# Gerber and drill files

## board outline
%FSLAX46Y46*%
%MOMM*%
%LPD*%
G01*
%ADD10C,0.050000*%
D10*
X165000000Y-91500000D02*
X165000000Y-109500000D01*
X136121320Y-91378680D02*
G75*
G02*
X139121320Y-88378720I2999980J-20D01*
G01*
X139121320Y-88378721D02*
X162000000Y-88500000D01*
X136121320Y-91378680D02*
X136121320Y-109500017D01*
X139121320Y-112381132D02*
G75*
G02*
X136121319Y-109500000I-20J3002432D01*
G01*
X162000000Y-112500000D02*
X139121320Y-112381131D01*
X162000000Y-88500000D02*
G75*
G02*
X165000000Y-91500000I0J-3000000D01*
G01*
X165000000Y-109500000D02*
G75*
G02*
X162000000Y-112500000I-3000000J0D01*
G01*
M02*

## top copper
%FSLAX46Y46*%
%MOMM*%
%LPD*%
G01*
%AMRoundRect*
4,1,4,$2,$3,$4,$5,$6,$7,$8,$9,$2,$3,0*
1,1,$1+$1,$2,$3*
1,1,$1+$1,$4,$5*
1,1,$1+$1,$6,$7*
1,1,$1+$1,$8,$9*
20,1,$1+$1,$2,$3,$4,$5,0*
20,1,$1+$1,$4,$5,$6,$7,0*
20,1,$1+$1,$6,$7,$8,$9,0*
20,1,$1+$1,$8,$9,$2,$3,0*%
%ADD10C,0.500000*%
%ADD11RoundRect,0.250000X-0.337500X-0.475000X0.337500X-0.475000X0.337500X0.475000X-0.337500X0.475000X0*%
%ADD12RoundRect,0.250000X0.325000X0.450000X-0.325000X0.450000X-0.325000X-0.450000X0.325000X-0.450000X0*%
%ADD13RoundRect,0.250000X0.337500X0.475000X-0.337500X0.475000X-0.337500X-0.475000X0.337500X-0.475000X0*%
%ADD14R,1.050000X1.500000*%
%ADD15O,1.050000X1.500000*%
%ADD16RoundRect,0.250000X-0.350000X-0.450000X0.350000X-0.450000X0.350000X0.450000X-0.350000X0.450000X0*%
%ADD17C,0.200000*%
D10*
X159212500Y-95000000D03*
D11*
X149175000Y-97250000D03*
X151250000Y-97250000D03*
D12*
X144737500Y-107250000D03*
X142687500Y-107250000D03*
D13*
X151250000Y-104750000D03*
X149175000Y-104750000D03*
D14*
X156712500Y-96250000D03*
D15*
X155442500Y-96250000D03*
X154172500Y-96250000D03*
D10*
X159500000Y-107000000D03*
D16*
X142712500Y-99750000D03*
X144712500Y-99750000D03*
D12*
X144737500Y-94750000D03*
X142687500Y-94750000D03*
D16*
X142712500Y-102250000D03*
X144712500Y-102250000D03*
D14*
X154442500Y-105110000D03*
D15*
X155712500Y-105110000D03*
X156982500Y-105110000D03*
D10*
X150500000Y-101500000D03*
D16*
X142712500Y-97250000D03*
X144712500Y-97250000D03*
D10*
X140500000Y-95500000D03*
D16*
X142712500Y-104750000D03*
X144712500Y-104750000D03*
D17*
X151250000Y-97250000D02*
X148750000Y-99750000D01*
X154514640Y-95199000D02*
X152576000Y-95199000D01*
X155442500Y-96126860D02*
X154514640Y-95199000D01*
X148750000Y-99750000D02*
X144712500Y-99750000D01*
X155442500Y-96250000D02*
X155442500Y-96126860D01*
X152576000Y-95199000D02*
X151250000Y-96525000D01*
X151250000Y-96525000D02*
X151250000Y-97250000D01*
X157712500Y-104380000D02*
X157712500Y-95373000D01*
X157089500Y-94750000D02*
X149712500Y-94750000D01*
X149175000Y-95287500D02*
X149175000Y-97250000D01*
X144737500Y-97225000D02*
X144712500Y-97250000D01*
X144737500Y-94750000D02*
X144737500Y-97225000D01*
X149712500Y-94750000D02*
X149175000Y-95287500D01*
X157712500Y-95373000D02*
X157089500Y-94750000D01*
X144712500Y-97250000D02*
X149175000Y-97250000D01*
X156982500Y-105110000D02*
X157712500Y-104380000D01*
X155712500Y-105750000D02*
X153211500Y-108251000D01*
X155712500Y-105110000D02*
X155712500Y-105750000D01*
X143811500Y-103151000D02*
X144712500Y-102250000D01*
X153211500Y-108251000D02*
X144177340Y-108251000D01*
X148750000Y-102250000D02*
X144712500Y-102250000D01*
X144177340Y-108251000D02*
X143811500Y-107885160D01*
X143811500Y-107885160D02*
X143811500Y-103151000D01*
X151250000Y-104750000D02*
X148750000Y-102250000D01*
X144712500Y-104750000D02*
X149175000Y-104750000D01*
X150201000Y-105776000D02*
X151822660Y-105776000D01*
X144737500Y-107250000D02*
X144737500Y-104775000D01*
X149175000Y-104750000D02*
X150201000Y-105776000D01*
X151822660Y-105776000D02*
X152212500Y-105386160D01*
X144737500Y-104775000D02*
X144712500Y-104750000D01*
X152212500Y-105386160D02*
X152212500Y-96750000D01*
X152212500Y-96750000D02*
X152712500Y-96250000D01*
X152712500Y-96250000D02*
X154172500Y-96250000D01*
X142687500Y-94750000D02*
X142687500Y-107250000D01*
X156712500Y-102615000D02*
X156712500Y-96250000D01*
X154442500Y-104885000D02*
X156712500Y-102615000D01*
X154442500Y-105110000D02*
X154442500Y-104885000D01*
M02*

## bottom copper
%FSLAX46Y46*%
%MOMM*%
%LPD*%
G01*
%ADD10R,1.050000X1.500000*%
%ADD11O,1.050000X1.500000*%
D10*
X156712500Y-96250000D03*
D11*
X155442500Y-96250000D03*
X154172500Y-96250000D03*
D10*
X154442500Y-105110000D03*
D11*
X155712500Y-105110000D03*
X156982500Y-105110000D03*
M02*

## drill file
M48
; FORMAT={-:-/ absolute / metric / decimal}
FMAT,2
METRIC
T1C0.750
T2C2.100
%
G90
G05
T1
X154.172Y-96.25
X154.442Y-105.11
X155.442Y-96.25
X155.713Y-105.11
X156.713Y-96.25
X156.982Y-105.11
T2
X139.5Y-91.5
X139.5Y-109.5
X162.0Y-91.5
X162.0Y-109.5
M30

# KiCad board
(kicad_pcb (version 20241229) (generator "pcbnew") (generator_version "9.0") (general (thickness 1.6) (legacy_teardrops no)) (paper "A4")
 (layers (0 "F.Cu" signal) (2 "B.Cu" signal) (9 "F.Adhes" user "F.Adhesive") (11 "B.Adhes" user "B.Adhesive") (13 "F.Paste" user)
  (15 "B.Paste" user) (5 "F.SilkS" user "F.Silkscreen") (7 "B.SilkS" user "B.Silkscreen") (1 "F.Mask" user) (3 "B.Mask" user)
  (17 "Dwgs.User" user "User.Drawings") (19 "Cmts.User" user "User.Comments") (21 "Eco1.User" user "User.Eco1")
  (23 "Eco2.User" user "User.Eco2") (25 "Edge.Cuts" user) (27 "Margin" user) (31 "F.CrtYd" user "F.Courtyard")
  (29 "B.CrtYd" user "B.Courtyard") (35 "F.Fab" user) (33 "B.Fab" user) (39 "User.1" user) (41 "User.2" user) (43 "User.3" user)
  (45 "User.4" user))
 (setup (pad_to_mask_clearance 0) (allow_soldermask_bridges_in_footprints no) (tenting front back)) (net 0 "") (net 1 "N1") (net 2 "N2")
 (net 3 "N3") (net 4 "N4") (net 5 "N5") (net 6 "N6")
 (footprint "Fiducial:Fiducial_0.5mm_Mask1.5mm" (layer "F.Cu") (at 159.2125 95)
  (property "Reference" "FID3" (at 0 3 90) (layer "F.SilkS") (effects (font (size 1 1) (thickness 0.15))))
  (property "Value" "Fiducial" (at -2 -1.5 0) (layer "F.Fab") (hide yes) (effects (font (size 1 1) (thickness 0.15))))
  (pad "" smd circle (at 0 0) (size 0.5 0.5) (layers "F.Cu" "F.Mask") (solder_mask_margin 0.5)))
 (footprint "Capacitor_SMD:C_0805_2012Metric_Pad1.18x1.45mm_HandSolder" (layer "F.Cu") (at 150.2125 97.25)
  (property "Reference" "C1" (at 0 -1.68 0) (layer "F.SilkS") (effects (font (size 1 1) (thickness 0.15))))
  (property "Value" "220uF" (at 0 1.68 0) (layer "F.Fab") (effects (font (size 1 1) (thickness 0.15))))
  (pad "1" smd roundrect (at -1.0375 0) (size 1.175 1.45) (layers "F.Cu" "F.Mask" "F.Paste") (roundrect_rratio 0.212766) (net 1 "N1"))
  (pad "2" smd roundrect (at 1.0375 0) (size 1.175 1.45) (layers "F.Cu" "F.Mask" "F.Paste") (roundrect_rratio 0.212766) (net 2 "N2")))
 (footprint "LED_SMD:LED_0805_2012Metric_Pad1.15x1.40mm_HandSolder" (layer "F.Cu") (at 143.7125 107.25 180)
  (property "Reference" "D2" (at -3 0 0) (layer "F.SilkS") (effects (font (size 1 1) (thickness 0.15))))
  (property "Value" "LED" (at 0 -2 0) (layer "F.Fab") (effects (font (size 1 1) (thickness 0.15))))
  (pad "1" smd roundrect (at -1.025 0 180) (size 1.15 1.4) (layers "F.Cu" "F.Mask" "F.Paste") (roundrect_rratio 0.217391) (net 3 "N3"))
  (pad "2" smd roundrect (at 1.025 0 180) (size 1.15 1.4) (layers "F.Cu" "F.Mask" "F.Paste") (roundrect_rratio 0.217391) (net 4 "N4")))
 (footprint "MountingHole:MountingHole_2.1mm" (layer "F.Cu") (at 162 91.5)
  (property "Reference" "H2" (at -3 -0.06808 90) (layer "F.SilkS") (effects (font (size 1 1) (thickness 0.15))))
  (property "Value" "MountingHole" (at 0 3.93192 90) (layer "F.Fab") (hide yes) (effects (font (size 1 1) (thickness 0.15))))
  (pad "" np_thru_hole circle (at 0 0) (size 2.1 2.1) (drill 2.1) (layers "*.Cu" "*.Mask")))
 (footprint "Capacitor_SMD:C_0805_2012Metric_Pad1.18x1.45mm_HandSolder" (layer "F.Cu") (at 150.2125 104.75 180)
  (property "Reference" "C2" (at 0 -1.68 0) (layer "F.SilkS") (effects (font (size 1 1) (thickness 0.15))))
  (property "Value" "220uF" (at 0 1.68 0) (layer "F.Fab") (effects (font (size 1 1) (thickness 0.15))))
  (pad "1" smd roundrect (at -1.0375 0 180) (size 1.175 1.45) (layers "F.Cu" "F.Mask" "F.Paste") (roundrect_rratio 0.212766) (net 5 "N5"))
  (pad "2" smd roundrect (at 1.0375 0 180) (size 1.175 1.45) (layers "F.Cu" "F.Mask" "F.Paste") (roundrect_rratio 0.212766) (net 3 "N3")))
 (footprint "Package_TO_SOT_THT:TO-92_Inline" (layer "F.Cu") (at 156.7125 96.25 180)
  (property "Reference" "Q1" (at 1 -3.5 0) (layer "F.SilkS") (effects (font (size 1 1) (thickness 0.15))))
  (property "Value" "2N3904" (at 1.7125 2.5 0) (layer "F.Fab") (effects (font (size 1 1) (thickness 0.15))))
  (pad "1" thru_hole rect (at 0 0 180) (size 1.05 1.5) (drill 0.75) (layers "*.Cu" "*.Mask") (remove_unused_layers no) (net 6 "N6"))
  (pad "2" thru_hole oval (at 1.27 0 180) (size 1.05 1.5) (drill 0.75) (layers "*.Cu" "*.Mask") (remove_unused_layers no) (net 2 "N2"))
  (pad "3" thru_hole oval (at 2.54 0 180) (size 1.05 1.5) (drill 0.75) (layers "*.Cu" "*.Mask") (remove_unused_layers no) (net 3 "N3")))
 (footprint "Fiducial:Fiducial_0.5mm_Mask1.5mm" (layer "F.Cu") (at 159.5 107)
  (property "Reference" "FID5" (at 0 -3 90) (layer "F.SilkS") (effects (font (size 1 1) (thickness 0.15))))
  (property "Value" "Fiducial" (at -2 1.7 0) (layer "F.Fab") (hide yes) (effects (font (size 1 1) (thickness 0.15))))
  (pad "" smd circle (at 0 0) (size 0.5 0.5) (layers "F.Cu" "F.Mask") (solder_mask_margin 0.5)))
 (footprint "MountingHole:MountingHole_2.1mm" (layer "F.Cu") (at 139.5 109.5)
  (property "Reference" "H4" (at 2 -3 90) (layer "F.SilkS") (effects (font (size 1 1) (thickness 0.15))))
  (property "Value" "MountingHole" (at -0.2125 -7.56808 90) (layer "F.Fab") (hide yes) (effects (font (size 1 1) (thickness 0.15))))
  (pad "" np_thru_hole circle (at 0 0) (size 2.1 2.1) (drill 2.1) (layers "*.Cu" "*.Mask")))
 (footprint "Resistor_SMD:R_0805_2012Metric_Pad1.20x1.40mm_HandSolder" (layer "F.Cu") (at 143.7125 99.75)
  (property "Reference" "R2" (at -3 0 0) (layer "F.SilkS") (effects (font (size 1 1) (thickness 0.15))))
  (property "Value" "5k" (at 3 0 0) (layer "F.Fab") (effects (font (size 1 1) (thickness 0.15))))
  (pad "1" smd roundrect (at -1 0) (size 1.2 1.4) (layers "F.Cu" "F.Mask" "F.Paste") (roundrect_rratio 0.208333) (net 4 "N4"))
  (pad "2" smd roundrect (at 1 0) (size 1.2 1.4) (layers "F.Cu" "F.Mask" "F.Paste") (roundrect_rratio 0.208333) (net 2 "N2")))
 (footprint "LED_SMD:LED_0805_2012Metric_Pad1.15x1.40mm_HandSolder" (layer "F.Cu") (at 143.7125 94.75 180)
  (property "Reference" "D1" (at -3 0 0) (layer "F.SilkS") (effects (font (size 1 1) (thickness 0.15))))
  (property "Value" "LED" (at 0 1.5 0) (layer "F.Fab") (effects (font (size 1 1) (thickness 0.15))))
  (pad "1" smd roundrect (at -1.025 0 180) (size 1.15 1.4) (layers "F.Cu" "F.Mask" "F.Paste") (roundrect_rratio 0.217391) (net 1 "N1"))
  (pad "2" smd roundrect (at 1.025 0 180) (size 1.15 1.4) (layers "F.Cu" "F.Mask" "F.Paste") (roundrect_rratio 0.217391) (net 4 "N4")))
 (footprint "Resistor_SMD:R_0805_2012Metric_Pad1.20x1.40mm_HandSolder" (layer "F.Cu") (at 143.7125 102.25)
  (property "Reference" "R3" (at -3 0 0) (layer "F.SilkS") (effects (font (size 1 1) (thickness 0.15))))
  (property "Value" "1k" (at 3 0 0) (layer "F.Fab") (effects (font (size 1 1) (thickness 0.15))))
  (pad "1" smd roundrect (at -1 0) (size 1.2 1.4) (layers "F.Cu" "F.Mask" "F.Paste") (roundrect_rratio 0.208333) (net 4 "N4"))
  (pad "2" smd roundrect (at 1 0) (size 1.2 1.4) (layers "F.Cu" "F.Mask" "F.Paste") (roundrect_rratio 0.208333) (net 5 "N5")))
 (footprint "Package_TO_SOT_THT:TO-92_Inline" (layer "F.Cu") (at 154.4425 105.11)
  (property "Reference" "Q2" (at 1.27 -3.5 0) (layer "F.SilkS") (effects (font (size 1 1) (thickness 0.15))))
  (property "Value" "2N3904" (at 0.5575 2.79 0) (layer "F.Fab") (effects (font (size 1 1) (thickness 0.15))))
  (pad "1" thru_hole rect (at 0 0) (size 1.05 1.5) (drill 0.75) (layers "*.Cu" "*.Mask") (remove_unused_layers no) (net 6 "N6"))
  (pad "2" thru_hole oval (at 1.27 0) (size 1.05 1.5) (drill 0.75) (layers "*.Cu" "*.Mask") (remove_unused_layers no) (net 5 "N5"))
  (pad "3" thru_hole oval (at 2.54 0) (size 1.05 1.5) (drill 0.75) (layers "*.Cu" "*.Mask") (remove_unused_layers no) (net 1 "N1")))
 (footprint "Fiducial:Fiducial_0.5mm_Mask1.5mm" (layer "F.Cu") (at 150.5 101.5)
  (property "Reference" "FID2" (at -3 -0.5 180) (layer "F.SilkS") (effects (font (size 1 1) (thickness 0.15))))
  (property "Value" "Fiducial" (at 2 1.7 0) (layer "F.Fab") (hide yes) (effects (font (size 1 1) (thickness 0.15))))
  (pad "" smd circle (at 0 0) (size 0.5 0.5) (layers "F.Cu" "F.Mask") (solder_mask_margin 0.5)))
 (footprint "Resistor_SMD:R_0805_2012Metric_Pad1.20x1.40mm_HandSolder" (layer "F.Cu") (at 143.7125 97.25)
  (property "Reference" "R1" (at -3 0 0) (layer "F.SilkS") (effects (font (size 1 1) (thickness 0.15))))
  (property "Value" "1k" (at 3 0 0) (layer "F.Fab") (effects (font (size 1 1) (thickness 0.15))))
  (pad "1" smd roundrect (at -1 0) (size 1.2 1.4) (layers "F.Cu" "F.Mask" "F.Paste") (roundrect_rratio 0.208333) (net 4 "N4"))
  (pad "2" smd roundrect (at 1 0) (size 1.2 1.4) (layers "F.Cu" "F.Mask" "F.Paste") (roundrect_rratio 0.208333) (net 1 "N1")))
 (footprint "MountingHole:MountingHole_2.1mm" (layer "F.Cu") (at 139.5 91.5)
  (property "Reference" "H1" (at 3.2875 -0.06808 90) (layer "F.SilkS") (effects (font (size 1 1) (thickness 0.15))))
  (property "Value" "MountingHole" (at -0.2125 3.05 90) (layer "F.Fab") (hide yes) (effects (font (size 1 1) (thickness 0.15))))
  (pad "" np_thru_hole circle (at 0 0) (size 2.1 2.1) (drill 2.1) (layers "*.Cu" "*.Mask")))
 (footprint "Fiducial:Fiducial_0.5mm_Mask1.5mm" (layer "F.Cu") (at 140.5 95.5)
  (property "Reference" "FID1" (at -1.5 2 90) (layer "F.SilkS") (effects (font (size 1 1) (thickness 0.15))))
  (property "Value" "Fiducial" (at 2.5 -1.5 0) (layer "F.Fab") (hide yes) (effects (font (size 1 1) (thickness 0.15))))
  (pad "" smd circle (at 0 0) (size 0.5 0.5) (layers "F.Cu" "F.Mask") (solder_mask_margin 0.5)))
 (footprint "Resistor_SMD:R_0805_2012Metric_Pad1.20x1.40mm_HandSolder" (layer "F.Cu") (at 143.7125 104.75)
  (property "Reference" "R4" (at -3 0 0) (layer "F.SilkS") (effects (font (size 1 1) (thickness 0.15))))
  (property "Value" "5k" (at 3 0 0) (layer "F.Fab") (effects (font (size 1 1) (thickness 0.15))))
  (pad "1" smd roundrect (at -1 0) (size 1.2 1.4) (layers "F.Cu" "F.Mask" "F.Paste") (roundrect_rratio 0.208333) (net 4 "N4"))
  (pad "2" smd roundrect (at 1 0) (size 1.2 1.4) (layers "F.Cu" "F.Mask" "F.Paste") (roundrect_rratio 0.208333) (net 3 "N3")))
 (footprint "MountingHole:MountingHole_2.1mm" (layer "F.Cu") (at 162 109.5)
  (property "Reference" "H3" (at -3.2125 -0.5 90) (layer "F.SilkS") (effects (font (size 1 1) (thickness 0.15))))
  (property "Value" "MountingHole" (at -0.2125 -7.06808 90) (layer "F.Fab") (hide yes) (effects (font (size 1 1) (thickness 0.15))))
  (pad "" np_thru_hole circle (at 0 0) (size 2.1 2.1) (drill 2.1) (layers "*.Cu" "*.Mask")))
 (gr_line (start 165 91.5) (end 165 109.5) (stroke (width 0.05) (type default)) (layer "Edge.Cuts"))
 (gr_arc (start 136.12132 91.37868) (mid 137 89.25736) (end 139.12132 88.37868) (stroke (width 0.05) (type default)) (layer "Edge.Cuts"))
 (gr_line (start 139.12132 88.378721) (end 162 88.5) (stroke (width 0.05) (type default)) (layer "Edge.Cuts"))
 (gr_line (start 136.12132 91.37868) (end 136.12132 109.500017) (stroke (width 0.05) (type default)) (layer "Edge.Cuts"))
 (gr_arc (start 139.12132 112.381132) (mid 137.041601 111.544203) (end 136.12132 109.5) (stroke (width 0.05) (type default))
  (layer "Edge.Cuts"))
 (gr_line (start 162 112.5) (end 139.12132 112.381131) (stroke (width 0.05) (type default)) (layer "Edge.Cuts"))
 (gr_arc (start 162 88.5) (mid 164.12132 89.37868) (end 165 91.5) (stroke (width 0.05) (type default)) (layer "Edge.Cuts"))
 (gr_arc (start 165 109.5) (mid 164.12132 111.62132) (end 162 112.5) (stroke (width 0.05) (type default)) (layer "Edge.Cuts"))
 (segment (start 151.25 97.25) (end 148.75 99.75) (width 0.2) (layer "F.Cu") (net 2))
 (segment (start 154.51464 95.199) (end 152.576 95.199) (width 0.2) (layer "F.Cu") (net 2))
 (segment (start 155.4425 96.12686) (end 154.51464 95.199) (width 0.2) (layer "F.Cu") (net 2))
 (segment (start 148.75 99.75) (end 144.7125 99.75) (width 0.2) (layer "F.Cu") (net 2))
 (segment (start 155.4425 96.25) (end 155.4425 96.12686) (width 0.2) (layer "F.Cu") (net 2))
 (segment (start 152.576 95.199) (end 151.25 96.525) (width 0.2) (layer "F.Cu") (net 2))
 (segment (start 151.25 96.525) (end 151.25 97.25) (width 0.2) (layer "F.Cu") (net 2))
 (segment (start 157.7125 104.38) (end 157.7125 95.373) (width 0.2) (layer "F.Cu") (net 1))
 (segment (start 157.0895 94.75) (end 149.7125 94.75) (width 0.2) (layer "F.Cu") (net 1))
 (segment (start 149.175 95.2875) (end 149.175 97.25) (width 0.2) (layer "F.Cu") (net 1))
 (segment (start 144.7375 97.225) (end 144.7125 97.25) (width 0.2) (layer "F.Cu") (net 1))
 (segment (start 144.7375 94.75) (end 144.7375 97.225) (width 0.2) (layer "F.Cu") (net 1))
 (segment (start 149.7125 94.75) (end 149.175 95.2875) (width 0.2) (layer "F.Cu") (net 1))
 (segment (start 157.7125 95.373) (end 157.0895 94.75) (width 0.2) (layer "F.Cu") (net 1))
 (segment (start 144.7125 97.25) (end 149.175 97.25) (width 0.2) (layer "F.Cu") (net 1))
 (segment (start 156.9825 105.11) (end 157.7125 104.38) (width 0.2) (layer "F.Cu") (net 1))
 (segment (start 155.7125 105.75) (end 153.2115 108.251) (width 0.2) (layer "F.Cu") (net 5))
 (segment (start 155.7125 105.11) (end 155.7125 105.75) (width 0.2) (layer "F.Cu") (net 5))
 (segment (start 143.8115 103.151) (end 144.7125 102.25) (width 0.2) (layer "F.Cu") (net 5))
 (segment (start 153.2115 108.251) (end 144.17734 108.251) (width 0.2) (layer "F.Cu") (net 5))
 (segment (start 148.75 102.25) (end 144.7125 102.25) (width 0.2) (layer "F.Cu") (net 5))
 (segment (start 144.17734 108.251) (end 143.8115 107.88516) (width 0.2) (layer "F.Cu") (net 5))
 (segment (start 143.8115 107.88516) (end 143.8115 103.151) (width 0.2) (layer "F.Cu") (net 5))
 (segment (start 151.25 104.75) (end 148.75 102.25) (width 0.2) (layer "F.Cu") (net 5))
 (segment (start 144.7125 104.75) (end 149.175 104.75) (width 0.2) (layer "F.Cu") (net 3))
 (segment (start 150.201 105.776) (end 151.82266 105.776) (width 0.2) (layer "F.Cu") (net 3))
 (segment (start 144.7375 107.25) (end 144.7375 104.775) (width 0.2) (layer "F.Cu") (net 3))
 (segment (start 149.175 104.75) (end 150.201 105.776) (width 0.2) (layer "F.Cu") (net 3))
 (segment (start 151.82266 105.776) (end 152.2125 105.38616) (width 0.2) (layer "F.Cu") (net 3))
 (segment (start 144.7375 104.775) (end 144.7125 104.75) (width 0.2) (layer "F.Cu") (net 3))
 (segment (start 152.2125 105.38616) (end 152.2125 96.75) (width 0.2) (layer "F.Cu") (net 3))
 (segment (start 152.2125 96.75) (end 152.7125 96.25) (width 0.2) (layer "F.Cu") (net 3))
 (segment (start 152.7125 96.25) (end 154.1725 96.25) (width 0.2) (layer "F.Cu") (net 3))
 (segment (start 142.6875 94.75) (end 142.6875 107.25) (width 0.2) (layer "F.Cu") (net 4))
 (segment (start 156.7125 102.615) (end 156.7125 96.25) (width 0.2) (layer "F.Cu") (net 6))
 (segment (start 154.4425 104.885) (end 156.7125 102.615) (width 0.2) (layer "F.Cu") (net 6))
 (segment (start 154.4425 105.11) (end 154.4425 104.885) (width 0.2) (layer "F.Cu") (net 6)))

